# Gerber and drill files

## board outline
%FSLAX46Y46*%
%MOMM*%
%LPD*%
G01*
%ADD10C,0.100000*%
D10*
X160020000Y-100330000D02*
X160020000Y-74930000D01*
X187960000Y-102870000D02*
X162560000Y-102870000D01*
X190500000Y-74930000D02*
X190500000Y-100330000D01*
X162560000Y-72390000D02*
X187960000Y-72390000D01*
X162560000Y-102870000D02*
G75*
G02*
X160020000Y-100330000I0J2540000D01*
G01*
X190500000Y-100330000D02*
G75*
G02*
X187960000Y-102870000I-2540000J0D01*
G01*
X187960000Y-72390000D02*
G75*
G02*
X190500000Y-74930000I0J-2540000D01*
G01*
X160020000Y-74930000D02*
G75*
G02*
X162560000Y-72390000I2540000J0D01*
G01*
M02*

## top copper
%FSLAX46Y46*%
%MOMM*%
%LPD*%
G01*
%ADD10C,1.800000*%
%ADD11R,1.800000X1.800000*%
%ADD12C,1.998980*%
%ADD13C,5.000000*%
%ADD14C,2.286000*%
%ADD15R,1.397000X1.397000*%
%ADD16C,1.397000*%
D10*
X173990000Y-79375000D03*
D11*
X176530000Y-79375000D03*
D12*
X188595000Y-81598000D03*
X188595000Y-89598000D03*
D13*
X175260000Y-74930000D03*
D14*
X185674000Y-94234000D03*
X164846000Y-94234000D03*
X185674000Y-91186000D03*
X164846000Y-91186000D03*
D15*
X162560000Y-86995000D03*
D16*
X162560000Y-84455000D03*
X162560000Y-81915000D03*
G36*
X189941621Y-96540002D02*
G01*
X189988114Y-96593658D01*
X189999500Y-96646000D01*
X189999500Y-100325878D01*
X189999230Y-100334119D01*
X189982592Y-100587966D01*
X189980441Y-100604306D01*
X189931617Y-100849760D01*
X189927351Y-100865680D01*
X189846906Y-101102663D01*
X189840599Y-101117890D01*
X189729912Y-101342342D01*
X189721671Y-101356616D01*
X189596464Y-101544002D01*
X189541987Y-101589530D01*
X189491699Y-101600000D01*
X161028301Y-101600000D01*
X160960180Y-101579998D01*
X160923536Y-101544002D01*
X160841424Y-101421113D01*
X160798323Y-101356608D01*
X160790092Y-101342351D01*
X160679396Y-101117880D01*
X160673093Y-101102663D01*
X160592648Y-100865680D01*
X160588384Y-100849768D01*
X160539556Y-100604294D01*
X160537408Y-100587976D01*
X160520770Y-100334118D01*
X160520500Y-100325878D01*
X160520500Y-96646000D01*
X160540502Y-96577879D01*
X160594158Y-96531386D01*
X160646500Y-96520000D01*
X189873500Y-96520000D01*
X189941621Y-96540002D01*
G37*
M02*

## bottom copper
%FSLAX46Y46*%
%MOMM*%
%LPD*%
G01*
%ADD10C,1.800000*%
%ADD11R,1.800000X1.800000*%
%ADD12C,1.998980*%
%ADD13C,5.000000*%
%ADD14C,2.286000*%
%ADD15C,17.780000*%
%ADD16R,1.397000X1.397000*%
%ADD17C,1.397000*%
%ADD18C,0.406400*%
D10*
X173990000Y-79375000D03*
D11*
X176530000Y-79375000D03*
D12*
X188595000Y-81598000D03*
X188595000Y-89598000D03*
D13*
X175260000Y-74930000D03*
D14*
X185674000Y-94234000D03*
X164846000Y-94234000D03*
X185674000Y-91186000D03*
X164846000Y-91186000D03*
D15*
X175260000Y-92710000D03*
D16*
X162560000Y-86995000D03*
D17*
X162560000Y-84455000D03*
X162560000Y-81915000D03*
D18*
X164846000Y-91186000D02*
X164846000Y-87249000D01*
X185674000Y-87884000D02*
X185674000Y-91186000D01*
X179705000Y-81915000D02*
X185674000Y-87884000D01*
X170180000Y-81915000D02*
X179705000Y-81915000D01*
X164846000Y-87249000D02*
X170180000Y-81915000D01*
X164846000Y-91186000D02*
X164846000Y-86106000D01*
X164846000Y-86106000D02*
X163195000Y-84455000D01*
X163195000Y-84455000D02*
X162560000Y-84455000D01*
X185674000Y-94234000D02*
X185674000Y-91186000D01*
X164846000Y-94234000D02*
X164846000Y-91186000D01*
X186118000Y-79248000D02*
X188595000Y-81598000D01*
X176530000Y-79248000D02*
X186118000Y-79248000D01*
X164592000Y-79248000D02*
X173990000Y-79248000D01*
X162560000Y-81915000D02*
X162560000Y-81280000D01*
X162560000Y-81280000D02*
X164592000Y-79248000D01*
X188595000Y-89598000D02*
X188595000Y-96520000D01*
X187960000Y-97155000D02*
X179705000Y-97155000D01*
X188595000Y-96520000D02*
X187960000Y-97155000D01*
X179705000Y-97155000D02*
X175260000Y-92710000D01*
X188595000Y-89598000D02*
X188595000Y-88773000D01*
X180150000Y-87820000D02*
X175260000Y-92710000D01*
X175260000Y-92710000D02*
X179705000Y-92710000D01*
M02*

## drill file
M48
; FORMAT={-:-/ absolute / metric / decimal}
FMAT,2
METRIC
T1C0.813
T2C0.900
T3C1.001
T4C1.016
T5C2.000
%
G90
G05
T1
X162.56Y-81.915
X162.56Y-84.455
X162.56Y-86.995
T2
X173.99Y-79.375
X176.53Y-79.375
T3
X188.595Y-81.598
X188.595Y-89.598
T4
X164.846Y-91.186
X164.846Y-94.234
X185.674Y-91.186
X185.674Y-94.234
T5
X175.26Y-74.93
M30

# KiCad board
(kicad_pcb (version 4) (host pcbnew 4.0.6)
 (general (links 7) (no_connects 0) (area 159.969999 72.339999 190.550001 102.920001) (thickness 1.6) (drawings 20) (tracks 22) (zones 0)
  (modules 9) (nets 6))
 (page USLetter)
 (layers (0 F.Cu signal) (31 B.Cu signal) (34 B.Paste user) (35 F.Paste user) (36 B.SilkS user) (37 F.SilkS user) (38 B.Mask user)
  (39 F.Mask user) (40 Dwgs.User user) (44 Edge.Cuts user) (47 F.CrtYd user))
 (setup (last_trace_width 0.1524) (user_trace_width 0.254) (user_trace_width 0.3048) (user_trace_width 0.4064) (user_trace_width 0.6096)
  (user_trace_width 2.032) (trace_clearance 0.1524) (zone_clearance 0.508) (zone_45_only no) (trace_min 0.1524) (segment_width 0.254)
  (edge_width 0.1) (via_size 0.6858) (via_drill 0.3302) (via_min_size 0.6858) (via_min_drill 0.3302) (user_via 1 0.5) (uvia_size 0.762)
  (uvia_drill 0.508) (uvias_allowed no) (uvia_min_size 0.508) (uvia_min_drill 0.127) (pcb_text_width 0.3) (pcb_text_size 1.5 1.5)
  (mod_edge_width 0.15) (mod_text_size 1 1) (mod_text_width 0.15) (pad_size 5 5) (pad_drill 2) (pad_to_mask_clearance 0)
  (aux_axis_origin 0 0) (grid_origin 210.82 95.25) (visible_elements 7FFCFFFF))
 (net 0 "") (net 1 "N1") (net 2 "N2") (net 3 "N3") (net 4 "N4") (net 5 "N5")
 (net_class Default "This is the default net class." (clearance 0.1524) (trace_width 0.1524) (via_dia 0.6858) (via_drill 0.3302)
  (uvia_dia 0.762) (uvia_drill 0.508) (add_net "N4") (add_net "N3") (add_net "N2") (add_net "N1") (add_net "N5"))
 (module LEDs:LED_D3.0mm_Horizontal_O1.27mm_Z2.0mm (layer F.Cu) (at 173.99 79.375)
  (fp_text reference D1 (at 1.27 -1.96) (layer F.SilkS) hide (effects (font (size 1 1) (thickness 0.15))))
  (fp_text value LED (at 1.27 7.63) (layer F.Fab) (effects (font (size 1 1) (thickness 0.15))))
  (pad 2 thru_hole circle (at 0 0) (size 1.8 1.8) (drill 0.9) (layers *.Cu *.Mask) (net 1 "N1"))
  (pad 1 thru_hole rect (at 2.54 0) (size 1.8 1.8) (drill 0.9) (layers *.Cu *.Mask) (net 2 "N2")))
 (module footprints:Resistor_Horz (layer F.Cu) (at 188.595 85.598 270)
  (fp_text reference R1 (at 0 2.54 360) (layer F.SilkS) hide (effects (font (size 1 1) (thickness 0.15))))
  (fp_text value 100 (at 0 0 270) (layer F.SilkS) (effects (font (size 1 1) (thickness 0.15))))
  (pad 1 thru_hole circle (at -4 0 270) (size 1.99898 1.99898) (drill 1.00076) (layers *.Cu *.SilkS *.Mask) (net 2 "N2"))
  (pad 2 thru_hole circle (at 4 0 270) (size 1.99898 1.99898) (drill 1.00076) (layers *.Cu *.SilkS *.Mask) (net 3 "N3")))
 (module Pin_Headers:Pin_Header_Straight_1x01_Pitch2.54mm (layer F.Cu) (at 175.26 74.93)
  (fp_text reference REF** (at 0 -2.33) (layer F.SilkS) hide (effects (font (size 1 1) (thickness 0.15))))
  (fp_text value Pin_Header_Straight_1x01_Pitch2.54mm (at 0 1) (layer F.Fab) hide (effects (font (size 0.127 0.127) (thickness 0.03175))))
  (pad 1 thru_hole circle (at 0 0) (size 5 5) (drill 2) (layers *.Cu *.Mask)))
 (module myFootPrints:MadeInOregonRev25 (layer F.Cu) (at 167.64 76.454)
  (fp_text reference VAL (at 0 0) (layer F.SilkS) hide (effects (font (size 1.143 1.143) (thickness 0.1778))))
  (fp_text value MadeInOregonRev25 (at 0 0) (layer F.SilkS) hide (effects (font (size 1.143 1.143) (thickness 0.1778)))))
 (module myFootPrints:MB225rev (layer F.Cu) (at 184.15 76.2)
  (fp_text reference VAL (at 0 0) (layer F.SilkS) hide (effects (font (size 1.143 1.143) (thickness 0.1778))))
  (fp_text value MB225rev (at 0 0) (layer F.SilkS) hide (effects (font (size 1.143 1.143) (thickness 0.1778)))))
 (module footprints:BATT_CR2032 (layer B.Cu) (at 175.26 92.71 180)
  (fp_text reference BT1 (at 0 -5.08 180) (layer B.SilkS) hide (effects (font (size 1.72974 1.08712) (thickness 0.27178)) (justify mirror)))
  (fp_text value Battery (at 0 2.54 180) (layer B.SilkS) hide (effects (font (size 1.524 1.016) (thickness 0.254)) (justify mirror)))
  (pad 1 thru_hole circle (at -10.414 -1.524 180) (size 2.286 2.286) (drill 1.016) (layers *.Cu *.Mask B.SilkS) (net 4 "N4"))
  (pad 1 thru_hole circle (at 10.414 -1.524 180) (size 2.286 2.286) (drill 1.016) (layers *.Cu *.Mask B.SilkS) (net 4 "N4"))
  (pad 1 thru_hole circle (at -10.414 1.524 180) (size 2.286 2.286) (drill 1.016) (layers *.Cu *.Mask B.SilkS) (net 4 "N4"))
  (pad 1 thru_hole circle (at 10.414 1.524 180) (size 2.286 2.286) (drill 1.016) (layers *.Cu *.Mask B.SilkS) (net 4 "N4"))
  (pad 2 smd circle (at 0 0 180) (size 17.78 17.78) (layers B.Cu B.Paste B.Mask) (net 3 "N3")))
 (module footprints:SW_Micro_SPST (layer F.Cu) (at 162.56 84.455 90)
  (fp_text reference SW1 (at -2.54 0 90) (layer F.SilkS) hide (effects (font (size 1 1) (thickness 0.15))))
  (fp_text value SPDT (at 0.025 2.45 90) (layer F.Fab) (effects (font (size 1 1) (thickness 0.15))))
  (pad 1 thru_hole rect (at -2.54 0 90) (size 1.397 1.397) (drill 0.8128) (layers *.Cu *.Mask F.SilkS) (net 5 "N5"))
  (pad 2 thru_hole circle (at 0 0 90) (size 1.397 1.397) (drill 0.8128) (layers *.Cu *.Mask F.SilkS) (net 4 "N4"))
  (pad 3 thru_hole circle (at 2.54 0 90) (size 1.397 1.397) (drill 0.8128) (layers *.Cu *.Mask F.SilkS) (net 1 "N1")))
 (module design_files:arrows (layer F.Cu) (at 177.546 81.788)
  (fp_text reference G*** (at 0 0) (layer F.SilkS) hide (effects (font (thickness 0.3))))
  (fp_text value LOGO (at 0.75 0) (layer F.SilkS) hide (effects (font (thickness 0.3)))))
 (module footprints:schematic (layer F.Cu) (at 175.26 87.503)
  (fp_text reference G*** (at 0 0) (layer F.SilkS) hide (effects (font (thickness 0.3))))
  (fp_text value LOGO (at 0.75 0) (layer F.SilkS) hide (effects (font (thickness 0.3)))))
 (gr_line (start 160.02 100.33) (end 160.02 74.93) (angle 90) (layer Edge.Cuts) (width 0.1))
 (gr_line (start 187.96 102.87) (end 162.56 102.87) (angle 90) (layer Edge.Cuts) (width 0.1))
 (gr_line (start 190.5 74.93) (end 190.5 100.33) (angle 90) (layer Edge.Cuts) (width 0.1))
 (gr_line (start 162.56 72.39) (end 187.96 72.39) (angle 90) (layer Edge.Cuts) (width 0.1))
 (gr_arc (start 162.56 100.33) (end 162.56 102.87) (angle 90) (layer Edge.Cuts) (width 0.1))
 (gr_arc (start 187.96 100.33) (end 190.5 100.33) (angle 90) (layer Edge.Cuts) (width 0.1))
 (gr_arc (start 187.96 74.93) (end 187.96 72.39) (angle 90) (layer Edge.Cuts) (width 0.1))
 (gr_arc (start 162.56 74.93) (end 160.02 74.93) (angle 90) (layer Edge.Cuts) (width 0.1))
 (segment (start 164.846 91.186) (end 164.846 87.249) (width 0.4064) (layer B.Cu) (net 4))
 (segment (start 185.674 87.884) (end 185.674 91.186) (width 0.4064) (layer B.Cu) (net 4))
 (segment (start 179.705 81.915) (end 185.674 87.884) (width 0.4064) (layer B.Cu) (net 4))
 (segment (start 170.18 81.915) (end 179.705 81.915) (width 0.4064) (layer B.Cu) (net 4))
 (segment (start 164.846 87.249) (end 170.18 81.915) (width 0.4064) (layer B.Cu) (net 4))
 (segment (start 164.846 91.186) (end 164.846 86.106) (width 0.4064) (layer B.Cu) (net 4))
 (segment (start 164.846 86.106) (end 163.195 84.455) (width 0.4064) (layer B.Cu) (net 4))
 (segment (start 163.195 84.455) (end 162.56 84.455) (width 0.4064) (layer B.Cu) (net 4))
 (segment (start 185.674 94.234) (end 185.674 91.186) (width 0.4064) (layer B.Cu) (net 4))
 (segment (start 164.846 94.234) (end 164.846 91.186) (width 0.4064) (layer B.Cu) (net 4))
 (segment (start 186.118 79.248) (end 188.595 81.598) (width 0.4064) (layer B.Cu) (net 2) (status 20))
 (segment (start 176.53 79.248) (end 186.118 79.248) (width 0.4064) (layer B.Cu) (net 2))
 (segment (start 164.592 79.248) (end 173.99 79.248) (width 0.4064) (layer B.Cu) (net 1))
 (segment (start 162.56 81.915) (end 162.56 81.28) (width 0.4064) (layer B.Cu) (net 1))
 (segment (start 162.56 81.28) (end 164.592 79.248) (width 0.4064) (layer B.Cu) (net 1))
 (segment (start 188.595 89.598) (end 188.595 96.52) (width 0.4064) (layer B.Cu) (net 3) (status 10))
 (segment (start 187.96 97.155) (end 179.705 97.155) (width 0.4064) (layer B.Cu) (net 3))
 (segment (start 188.595 96.52) (end 187.96 97.155) (width 0.4064) (layer B.Cu) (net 3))
 (segment (start 179.705 97.155) (end 175.26 92.71) (width 0.4064) (layer B.Cu) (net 3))
 (segment (start 188.595 89.598) (end 188.595 88.773) (width 0.4064) (layer B.Cu) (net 3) (status 30))
 (segment (start 180.15 87.82) (end 175.26 92.71) (width 0.4064) (layer B.Cu) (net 3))
 (segment (start 175.26 92.71) (end 179.705 92.71) (width 0.4064) (layer B.Cu) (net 3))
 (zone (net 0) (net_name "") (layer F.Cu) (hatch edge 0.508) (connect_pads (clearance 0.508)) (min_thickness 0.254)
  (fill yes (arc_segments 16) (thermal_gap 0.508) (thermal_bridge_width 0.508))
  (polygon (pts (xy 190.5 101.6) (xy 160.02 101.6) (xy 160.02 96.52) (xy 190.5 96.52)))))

